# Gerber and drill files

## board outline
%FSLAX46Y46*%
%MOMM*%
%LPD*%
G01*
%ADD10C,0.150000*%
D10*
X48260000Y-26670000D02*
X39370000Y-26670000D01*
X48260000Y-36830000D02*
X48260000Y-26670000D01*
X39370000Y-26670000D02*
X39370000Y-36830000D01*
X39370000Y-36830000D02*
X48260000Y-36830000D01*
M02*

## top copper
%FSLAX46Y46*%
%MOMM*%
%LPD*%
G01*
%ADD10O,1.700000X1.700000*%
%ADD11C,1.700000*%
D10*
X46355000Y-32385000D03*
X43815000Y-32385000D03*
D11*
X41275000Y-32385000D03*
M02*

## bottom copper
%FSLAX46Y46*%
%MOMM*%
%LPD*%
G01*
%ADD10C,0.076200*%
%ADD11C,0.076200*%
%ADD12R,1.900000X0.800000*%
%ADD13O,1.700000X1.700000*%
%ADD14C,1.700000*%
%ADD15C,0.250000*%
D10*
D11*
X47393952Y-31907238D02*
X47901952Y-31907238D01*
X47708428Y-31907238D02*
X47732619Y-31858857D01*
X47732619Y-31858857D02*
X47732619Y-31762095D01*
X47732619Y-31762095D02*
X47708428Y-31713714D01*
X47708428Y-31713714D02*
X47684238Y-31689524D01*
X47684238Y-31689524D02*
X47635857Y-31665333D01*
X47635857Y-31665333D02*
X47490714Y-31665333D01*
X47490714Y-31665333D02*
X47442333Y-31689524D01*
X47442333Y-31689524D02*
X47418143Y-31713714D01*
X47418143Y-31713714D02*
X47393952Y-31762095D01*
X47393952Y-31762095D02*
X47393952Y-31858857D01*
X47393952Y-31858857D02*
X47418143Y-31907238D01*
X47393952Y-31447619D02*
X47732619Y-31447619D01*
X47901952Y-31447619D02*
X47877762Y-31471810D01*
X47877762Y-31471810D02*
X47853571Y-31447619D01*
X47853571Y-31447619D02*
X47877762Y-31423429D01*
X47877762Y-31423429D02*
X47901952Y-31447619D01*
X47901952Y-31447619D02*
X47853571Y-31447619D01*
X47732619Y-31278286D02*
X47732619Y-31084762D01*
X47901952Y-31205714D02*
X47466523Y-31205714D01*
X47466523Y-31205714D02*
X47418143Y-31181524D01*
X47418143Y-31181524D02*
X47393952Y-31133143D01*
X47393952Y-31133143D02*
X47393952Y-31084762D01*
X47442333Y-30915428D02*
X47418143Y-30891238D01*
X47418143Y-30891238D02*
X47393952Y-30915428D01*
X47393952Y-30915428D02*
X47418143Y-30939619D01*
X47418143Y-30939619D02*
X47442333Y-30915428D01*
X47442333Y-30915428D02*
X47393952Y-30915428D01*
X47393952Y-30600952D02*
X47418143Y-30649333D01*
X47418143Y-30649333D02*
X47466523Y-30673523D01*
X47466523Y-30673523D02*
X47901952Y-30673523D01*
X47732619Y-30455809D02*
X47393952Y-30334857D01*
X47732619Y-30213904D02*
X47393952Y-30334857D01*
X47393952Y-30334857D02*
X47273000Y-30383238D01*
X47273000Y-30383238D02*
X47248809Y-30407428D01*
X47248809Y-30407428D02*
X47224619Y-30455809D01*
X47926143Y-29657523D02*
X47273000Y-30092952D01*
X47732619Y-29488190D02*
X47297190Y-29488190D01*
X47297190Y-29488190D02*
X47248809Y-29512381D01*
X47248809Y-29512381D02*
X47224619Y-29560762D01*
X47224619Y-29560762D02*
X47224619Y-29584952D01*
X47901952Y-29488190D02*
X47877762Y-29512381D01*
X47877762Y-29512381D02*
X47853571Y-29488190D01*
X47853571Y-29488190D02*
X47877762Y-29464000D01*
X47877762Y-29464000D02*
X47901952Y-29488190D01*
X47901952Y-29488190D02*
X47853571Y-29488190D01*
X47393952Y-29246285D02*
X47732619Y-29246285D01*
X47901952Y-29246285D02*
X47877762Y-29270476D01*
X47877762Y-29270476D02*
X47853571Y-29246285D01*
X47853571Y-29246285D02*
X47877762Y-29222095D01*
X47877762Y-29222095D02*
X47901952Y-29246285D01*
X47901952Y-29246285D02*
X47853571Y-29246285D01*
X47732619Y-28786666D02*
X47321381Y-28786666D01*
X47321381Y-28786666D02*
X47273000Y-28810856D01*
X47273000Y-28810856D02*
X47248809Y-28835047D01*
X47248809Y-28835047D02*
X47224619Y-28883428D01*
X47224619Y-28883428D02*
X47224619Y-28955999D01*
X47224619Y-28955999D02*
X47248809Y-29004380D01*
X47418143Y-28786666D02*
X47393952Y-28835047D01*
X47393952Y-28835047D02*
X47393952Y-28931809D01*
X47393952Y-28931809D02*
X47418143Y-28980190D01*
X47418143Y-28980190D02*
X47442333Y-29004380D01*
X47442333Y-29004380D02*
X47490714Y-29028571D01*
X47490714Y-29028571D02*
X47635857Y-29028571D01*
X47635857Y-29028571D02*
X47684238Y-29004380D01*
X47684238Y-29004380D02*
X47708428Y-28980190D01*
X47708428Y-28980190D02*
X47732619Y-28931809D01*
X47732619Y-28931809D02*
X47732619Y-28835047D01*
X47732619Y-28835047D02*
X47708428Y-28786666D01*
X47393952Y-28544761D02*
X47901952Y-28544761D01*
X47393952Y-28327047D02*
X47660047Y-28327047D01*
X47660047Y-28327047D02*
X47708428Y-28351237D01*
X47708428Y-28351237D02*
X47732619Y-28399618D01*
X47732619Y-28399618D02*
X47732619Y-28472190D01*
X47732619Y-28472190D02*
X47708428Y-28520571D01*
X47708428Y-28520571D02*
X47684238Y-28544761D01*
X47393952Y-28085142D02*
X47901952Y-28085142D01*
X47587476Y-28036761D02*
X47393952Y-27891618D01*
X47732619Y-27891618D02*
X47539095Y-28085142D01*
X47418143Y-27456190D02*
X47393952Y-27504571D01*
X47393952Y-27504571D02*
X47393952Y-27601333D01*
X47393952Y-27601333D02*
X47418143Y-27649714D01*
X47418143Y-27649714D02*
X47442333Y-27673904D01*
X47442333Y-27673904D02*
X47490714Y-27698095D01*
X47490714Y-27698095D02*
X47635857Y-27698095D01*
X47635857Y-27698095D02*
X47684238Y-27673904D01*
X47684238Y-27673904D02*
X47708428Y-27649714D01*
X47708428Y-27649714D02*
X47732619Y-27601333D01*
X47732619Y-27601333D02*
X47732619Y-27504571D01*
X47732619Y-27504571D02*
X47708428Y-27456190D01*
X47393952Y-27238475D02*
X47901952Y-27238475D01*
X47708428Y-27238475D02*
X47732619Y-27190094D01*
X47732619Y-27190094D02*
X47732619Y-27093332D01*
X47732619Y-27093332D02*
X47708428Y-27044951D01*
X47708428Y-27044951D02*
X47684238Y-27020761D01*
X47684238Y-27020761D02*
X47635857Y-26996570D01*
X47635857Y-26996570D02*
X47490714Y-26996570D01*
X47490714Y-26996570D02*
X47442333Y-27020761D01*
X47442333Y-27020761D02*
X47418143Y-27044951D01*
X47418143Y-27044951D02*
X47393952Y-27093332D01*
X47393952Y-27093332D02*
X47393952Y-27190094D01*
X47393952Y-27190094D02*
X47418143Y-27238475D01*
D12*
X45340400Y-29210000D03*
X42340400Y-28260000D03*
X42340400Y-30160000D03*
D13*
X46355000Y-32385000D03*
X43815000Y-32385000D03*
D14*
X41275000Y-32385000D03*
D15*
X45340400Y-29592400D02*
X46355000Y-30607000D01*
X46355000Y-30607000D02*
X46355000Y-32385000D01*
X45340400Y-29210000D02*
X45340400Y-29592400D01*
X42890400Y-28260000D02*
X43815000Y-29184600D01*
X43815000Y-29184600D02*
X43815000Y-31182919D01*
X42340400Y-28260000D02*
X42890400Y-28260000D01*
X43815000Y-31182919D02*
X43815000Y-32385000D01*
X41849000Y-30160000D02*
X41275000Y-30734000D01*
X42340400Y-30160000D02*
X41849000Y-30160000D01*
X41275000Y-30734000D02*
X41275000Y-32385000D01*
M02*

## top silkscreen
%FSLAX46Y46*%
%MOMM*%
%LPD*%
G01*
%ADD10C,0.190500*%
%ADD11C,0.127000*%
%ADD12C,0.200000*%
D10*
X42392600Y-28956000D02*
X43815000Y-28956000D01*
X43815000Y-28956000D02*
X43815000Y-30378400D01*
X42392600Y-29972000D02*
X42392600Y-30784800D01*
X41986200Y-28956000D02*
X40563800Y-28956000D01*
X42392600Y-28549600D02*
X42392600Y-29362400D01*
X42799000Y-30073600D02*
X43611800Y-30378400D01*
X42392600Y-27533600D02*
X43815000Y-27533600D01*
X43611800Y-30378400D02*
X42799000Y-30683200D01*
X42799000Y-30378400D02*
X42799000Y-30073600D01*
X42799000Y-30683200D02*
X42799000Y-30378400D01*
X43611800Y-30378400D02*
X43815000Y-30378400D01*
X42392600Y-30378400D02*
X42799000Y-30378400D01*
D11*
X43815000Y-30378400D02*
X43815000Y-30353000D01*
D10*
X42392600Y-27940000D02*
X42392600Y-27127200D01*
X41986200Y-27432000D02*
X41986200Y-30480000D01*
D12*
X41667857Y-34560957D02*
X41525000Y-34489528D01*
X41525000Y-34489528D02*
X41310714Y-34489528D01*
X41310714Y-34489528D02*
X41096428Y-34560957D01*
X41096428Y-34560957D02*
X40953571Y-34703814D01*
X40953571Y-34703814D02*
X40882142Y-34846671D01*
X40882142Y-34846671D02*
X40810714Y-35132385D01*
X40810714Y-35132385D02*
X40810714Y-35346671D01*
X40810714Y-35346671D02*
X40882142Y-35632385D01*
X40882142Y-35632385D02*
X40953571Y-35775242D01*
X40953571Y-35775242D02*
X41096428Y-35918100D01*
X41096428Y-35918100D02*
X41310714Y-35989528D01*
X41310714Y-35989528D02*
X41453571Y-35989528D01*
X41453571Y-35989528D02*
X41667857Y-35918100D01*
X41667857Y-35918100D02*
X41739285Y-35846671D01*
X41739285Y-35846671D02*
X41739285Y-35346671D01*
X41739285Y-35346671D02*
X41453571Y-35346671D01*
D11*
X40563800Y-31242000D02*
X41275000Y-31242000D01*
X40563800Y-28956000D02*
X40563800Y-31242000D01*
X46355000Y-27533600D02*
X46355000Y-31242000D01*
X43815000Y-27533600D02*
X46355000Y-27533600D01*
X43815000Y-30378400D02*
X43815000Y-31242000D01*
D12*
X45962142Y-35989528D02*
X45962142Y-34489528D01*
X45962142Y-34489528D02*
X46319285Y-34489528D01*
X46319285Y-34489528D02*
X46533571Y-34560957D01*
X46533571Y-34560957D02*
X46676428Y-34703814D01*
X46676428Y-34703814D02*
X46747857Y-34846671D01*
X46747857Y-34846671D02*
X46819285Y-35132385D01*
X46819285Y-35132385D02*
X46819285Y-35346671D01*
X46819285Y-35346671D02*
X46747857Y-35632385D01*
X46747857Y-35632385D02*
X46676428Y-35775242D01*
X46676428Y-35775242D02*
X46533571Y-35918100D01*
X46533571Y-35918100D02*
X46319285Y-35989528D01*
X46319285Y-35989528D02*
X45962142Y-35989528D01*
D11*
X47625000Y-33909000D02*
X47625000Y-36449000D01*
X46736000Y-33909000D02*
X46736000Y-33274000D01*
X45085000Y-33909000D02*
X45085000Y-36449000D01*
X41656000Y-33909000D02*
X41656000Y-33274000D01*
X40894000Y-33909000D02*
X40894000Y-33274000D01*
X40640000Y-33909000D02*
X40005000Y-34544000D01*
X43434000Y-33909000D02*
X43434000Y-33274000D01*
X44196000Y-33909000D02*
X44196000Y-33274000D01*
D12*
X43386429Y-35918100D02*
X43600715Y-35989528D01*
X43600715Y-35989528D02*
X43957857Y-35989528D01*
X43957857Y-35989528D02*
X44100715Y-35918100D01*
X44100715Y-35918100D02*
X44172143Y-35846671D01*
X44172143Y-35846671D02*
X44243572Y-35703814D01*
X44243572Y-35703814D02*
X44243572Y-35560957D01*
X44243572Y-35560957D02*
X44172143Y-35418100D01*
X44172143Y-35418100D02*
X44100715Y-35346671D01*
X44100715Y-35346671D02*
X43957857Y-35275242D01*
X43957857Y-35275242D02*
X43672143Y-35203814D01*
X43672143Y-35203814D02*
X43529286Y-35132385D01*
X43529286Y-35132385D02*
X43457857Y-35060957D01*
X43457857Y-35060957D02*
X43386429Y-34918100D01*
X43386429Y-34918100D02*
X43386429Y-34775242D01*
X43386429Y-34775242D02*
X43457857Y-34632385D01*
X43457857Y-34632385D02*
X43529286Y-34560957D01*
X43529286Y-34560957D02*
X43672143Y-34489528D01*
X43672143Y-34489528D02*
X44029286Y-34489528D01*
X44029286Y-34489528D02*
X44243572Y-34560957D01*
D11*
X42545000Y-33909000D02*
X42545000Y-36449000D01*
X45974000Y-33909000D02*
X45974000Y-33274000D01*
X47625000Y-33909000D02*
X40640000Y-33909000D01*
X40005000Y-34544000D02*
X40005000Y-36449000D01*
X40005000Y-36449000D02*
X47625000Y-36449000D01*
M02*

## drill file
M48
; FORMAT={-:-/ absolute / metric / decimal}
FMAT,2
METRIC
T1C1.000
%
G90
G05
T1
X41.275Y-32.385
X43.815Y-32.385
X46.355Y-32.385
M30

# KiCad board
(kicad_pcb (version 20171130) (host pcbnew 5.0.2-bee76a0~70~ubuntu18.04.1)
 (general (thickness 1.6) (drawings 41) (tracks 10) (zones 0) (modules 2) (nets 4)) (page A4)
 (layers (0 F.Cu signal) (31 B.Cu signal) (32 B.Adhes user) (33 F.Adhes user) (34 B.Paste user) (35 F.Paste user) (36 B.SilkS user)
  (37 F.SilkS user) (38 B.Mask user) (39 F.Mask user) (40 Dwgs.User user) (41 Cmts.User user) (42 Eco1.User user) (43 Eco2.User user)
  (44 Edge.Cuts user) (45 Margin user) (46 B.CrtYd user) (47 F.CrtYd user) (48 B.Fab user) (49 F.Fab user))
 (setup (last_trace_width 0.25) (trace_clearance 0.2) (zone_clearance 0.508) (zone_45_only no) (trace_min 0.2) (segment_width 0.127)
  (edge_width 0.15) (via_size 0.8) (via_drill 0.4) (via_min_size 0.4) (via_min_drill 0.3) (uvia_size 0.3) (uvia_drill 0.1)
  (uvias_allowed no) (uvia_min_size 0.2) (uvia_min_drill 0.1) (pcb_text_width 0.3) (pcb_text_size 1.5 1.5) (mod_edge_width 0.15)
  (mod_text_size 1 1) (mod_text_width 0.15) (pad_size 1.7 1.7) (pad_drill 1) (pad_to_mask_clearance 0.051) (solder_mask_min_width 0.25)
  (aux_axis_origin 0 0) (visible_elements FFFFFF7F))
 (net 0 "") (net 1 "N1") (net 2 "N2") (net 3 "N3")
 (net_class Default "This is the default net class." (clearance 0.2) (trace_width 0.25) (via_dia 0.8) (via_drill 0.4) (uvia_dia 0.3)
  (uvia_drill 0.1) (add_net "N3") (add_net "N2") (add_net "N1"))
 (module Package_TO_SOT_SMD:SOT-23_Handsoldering (layer B.Cu) (at 43.8404 29.21)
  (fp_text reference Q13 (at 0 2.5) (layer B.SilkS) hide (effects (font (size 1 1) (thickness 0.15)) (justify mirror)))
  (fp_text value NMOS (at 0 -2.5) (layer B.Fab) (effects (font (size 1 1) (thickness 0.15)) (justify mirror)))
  (pad 3 smd rect (at 1.5 0) (size 1.9 0.8) (layers B.Cu B.Paste B.Mask) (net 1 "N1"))
  (pad 2 smd rect (at -1.5 -0.95) (size 1.9 0.8) (layers B.Cu B.Paste B.Mask) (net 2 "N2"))
  (pad 1 smd rect (at -1.5 0.95) (size 1.9 0.8) (layers B.Cu B.Paste B.Mask) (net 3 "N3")))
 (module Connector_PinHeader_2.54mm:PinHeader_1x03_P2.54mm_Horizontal (layer B.Cu) (at 41.275 32.385 270)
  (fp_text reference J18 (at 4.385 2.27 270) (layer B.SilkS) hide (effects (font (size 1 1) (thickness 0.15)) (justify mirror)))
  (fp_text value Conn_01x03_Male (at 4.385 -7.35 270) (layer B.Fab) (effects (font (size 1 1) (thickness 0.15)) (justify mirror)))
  (pad 3 thru_hole oval (at 0 -5.08 270) (size 1.7 1.7) (drill 1) (layers *.Cu *.Mask) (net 1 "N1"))
  (pad 2 thru_hole oval (at 0 -2.54 270) (size 1.7 1.7) (drill 1) (layers *.Cu *.Mask) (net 2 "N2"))
  (pad 1 thru_hole circle (at 0 0 270) (size 1.7 1.7) (drill 1) (layers *.Cu *.Mask) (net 3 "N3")))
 (gr_line (start 42.3926 28.956) (end 43.815 28.956) (layer F.SilkS) (width 0.1905))
 (gr_line (start 43.815 28.956) (end 43.815 30.3784) (layer F.SilkS) (width 0.1905))
 (gr_line (start 42.3926 29.972) (end 42.3926 30.7848) (layer F.SilkS) (width 0.1905))
 (gr_line (start 41.9862 28.956) (end 40.5638 28.956) (layer F.SilkS) (width 0.1905))
 (gr_line (start 42.3926 28.5496) (end 42.3926 29.3624) (layer F.SilkS) (width 0.1905))
 (gr_line (start 42.799 30.0736) (end 43.6118 30.3784) (layer F.SilkS) (width 0.1905))
 (gr_line (start 42.3926 27.5336) (end 43.815 27.5336) (layer F.SilkS) (width 0.1905))
 (gr_line (start 43.6118 30.3784) (end 42.799 30.6832) (layer F.SilkS) (width 0.1905))
 (gr_line (start 42.799 30.3784) (end 42.799 30.0736) (layer F.SilkS) (width 0.1905))
 (gr_line (start 42.799 30.6832) (end 42.799 30.3784) (layer F.SilkS) (width 0.1905))
 (gr_line (start 43.6118 30.3784) (end 43.815 30.3784) (layer F.SilkS) (width 0.1905))
 (gr_line (start 42.3926 30.3784) (end 42.799 30.3784) (layer F.SilkS) (width 0.1905))
 (gr_line (start 43.815 30.3784) (end 43.815 30.353) (layer F.SilkS) (width 0.127))
 (gr_line (start 42.3926 27.94) (end 42.3926 27.1272) (layer F.SilkS) (width 0.1905))
 (gr_line (start 41.9862 27.432) (end 41.9862 30.48) (layer F.SilkS) (width 0.1905))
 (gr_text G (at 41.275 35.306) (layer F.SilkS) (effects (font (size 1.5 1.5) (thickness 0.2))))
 (gr_line (start 40.5638 31.242) (end 41.275 31.242) (layer F.SilkS) (width 0.127))
 (gr_line (start 40.5638 28.956) (end 40.5638 31.242) (layer F.SilkS) (width 0.127))
 (gr_line (start 46.355 27.5336) (end 46.355 31.242) (layer F.SilkS) (width 0.127))
 (gr_line (start 43.815 27.5336) (end 46.355 27.5336) (layer F.SilkS) (width 0.127))
 (gr_line (start 43.815 30.3784) (end 43.815 31.242) (layer F.SilkS) (width 0.127))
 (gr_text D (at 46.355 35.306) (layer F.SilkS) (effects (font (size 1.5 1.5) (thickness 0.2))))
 (gr_line (start 47.625 33.909) (end 47.625 36.449) (layer F.SilkS) (width 0.127))
 (gr_line (start 46.736 33.909) (end 46.736 33.274) (layer F.SilkS) (width 0.127))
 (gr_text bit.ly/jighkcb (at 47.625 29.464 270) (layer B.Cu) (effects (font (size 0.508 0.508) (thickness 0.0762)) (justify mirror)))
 (gr_line (start 45.085 33.909) (end 45.085 36.449) (layer F.SilkS) (width 0.127))
 (gr_line (start 41.656 33.909) (end 41.656 33.274) (layer F.SilkS) (width 0.127))
 (gr_line (start 40.894 33.909) (end 40.894 33.274) (layer F.SilkS) (width 0.127))
 (gr_line (start 40.64 33.909) (end 40.005 34.544) (layer F.SilkS) (width 0.127))
 (gr_line (start 43.434 33.909) (end 43.434 33.274) (layer F.SilkS) (width 0.127))
 (gr_line (start 48.26 26.67) (end 39.37 26.67) (layer Edge.Cuts) (width 0.15))
 (gr_line (start 44.196 33.909) (end 44.196 33.274) (layer F.SilkS) (width 0.127))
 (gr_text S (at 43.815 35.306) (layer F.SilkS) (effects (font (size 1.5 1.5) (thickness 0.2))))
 (gr_line (start 42.545 33.909) (end 42.545 36.449) (layer F.SilkS) (width 0.127))
 (gr_line (start 45.974 33.909) (end 45.974 33.274) (layer F.SilkS) (width 0.127))
 (gr_line (start 47.625 33.909) (end 40.64 33.909) (layer F.SilkS) (width 0.127))
 (gr_line (start 40.005 34.544) (end 40.005 36.449) (layer F.SilkS) (width 0.127))
 (gr_line (start 40.005 36.449) (end 47.625 36.449) (layer F.SilkS) (width 0.127))
 (gr_line (start 48.26 36.83) (end 48.26 26.67) (layer Edge.Cuts) (width 0.15))
 (gr_line (start 39.37 26.67) (end 39.37 36.83) (layer Edge.Cuts) (width 0.15))
 (gr_line (start 39.37 36.83) (end 48.26 36.83) (layer Edge.Cuts) (width 0.15))
 (segment (start 45.3404 29.5924) (end 46.355 30.607) (width 0.25) (layer B.Cu) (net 1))
 (segment (start 46.355 30.607) (end 46.355 32.385) (width 0.25) (layer B.Cu) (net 1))
 (segment (start 45.3404 29.21) (end 45.3404 29.5924) (width 0.25) (layer B.Cu) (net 1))
 (segment (start 42.8904 28.26) (end 43.815 29.1846) (width 0.25) (layer B.Cu) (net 2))
 (segment (start 43.815 29.1846) (end 43.815 31.182919) (width 0.25) (layer B.Cu) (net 2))
 (segment (start 42.3404 28.26) (end 42.8904 28.26) (width 0.25) (layer B.Cu) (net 2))
 (segment (start 43.815 31.182919) (end 43.815 32.385) (width 0.25) (layer B.Cu) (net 2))
 (segment (start 41.849 30.16) (end 41.275 30.734) (width 0.25) (layer B.Cu) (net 3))
 (segment (start 42.3404 30.16) (end 41.849 30.16) (width 0.25) (layer B.Cu) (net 3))
 (segment (start 41.275 30.734) (end 41.275 32.385) (width 0.25) (layer B.Cu) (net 3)))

